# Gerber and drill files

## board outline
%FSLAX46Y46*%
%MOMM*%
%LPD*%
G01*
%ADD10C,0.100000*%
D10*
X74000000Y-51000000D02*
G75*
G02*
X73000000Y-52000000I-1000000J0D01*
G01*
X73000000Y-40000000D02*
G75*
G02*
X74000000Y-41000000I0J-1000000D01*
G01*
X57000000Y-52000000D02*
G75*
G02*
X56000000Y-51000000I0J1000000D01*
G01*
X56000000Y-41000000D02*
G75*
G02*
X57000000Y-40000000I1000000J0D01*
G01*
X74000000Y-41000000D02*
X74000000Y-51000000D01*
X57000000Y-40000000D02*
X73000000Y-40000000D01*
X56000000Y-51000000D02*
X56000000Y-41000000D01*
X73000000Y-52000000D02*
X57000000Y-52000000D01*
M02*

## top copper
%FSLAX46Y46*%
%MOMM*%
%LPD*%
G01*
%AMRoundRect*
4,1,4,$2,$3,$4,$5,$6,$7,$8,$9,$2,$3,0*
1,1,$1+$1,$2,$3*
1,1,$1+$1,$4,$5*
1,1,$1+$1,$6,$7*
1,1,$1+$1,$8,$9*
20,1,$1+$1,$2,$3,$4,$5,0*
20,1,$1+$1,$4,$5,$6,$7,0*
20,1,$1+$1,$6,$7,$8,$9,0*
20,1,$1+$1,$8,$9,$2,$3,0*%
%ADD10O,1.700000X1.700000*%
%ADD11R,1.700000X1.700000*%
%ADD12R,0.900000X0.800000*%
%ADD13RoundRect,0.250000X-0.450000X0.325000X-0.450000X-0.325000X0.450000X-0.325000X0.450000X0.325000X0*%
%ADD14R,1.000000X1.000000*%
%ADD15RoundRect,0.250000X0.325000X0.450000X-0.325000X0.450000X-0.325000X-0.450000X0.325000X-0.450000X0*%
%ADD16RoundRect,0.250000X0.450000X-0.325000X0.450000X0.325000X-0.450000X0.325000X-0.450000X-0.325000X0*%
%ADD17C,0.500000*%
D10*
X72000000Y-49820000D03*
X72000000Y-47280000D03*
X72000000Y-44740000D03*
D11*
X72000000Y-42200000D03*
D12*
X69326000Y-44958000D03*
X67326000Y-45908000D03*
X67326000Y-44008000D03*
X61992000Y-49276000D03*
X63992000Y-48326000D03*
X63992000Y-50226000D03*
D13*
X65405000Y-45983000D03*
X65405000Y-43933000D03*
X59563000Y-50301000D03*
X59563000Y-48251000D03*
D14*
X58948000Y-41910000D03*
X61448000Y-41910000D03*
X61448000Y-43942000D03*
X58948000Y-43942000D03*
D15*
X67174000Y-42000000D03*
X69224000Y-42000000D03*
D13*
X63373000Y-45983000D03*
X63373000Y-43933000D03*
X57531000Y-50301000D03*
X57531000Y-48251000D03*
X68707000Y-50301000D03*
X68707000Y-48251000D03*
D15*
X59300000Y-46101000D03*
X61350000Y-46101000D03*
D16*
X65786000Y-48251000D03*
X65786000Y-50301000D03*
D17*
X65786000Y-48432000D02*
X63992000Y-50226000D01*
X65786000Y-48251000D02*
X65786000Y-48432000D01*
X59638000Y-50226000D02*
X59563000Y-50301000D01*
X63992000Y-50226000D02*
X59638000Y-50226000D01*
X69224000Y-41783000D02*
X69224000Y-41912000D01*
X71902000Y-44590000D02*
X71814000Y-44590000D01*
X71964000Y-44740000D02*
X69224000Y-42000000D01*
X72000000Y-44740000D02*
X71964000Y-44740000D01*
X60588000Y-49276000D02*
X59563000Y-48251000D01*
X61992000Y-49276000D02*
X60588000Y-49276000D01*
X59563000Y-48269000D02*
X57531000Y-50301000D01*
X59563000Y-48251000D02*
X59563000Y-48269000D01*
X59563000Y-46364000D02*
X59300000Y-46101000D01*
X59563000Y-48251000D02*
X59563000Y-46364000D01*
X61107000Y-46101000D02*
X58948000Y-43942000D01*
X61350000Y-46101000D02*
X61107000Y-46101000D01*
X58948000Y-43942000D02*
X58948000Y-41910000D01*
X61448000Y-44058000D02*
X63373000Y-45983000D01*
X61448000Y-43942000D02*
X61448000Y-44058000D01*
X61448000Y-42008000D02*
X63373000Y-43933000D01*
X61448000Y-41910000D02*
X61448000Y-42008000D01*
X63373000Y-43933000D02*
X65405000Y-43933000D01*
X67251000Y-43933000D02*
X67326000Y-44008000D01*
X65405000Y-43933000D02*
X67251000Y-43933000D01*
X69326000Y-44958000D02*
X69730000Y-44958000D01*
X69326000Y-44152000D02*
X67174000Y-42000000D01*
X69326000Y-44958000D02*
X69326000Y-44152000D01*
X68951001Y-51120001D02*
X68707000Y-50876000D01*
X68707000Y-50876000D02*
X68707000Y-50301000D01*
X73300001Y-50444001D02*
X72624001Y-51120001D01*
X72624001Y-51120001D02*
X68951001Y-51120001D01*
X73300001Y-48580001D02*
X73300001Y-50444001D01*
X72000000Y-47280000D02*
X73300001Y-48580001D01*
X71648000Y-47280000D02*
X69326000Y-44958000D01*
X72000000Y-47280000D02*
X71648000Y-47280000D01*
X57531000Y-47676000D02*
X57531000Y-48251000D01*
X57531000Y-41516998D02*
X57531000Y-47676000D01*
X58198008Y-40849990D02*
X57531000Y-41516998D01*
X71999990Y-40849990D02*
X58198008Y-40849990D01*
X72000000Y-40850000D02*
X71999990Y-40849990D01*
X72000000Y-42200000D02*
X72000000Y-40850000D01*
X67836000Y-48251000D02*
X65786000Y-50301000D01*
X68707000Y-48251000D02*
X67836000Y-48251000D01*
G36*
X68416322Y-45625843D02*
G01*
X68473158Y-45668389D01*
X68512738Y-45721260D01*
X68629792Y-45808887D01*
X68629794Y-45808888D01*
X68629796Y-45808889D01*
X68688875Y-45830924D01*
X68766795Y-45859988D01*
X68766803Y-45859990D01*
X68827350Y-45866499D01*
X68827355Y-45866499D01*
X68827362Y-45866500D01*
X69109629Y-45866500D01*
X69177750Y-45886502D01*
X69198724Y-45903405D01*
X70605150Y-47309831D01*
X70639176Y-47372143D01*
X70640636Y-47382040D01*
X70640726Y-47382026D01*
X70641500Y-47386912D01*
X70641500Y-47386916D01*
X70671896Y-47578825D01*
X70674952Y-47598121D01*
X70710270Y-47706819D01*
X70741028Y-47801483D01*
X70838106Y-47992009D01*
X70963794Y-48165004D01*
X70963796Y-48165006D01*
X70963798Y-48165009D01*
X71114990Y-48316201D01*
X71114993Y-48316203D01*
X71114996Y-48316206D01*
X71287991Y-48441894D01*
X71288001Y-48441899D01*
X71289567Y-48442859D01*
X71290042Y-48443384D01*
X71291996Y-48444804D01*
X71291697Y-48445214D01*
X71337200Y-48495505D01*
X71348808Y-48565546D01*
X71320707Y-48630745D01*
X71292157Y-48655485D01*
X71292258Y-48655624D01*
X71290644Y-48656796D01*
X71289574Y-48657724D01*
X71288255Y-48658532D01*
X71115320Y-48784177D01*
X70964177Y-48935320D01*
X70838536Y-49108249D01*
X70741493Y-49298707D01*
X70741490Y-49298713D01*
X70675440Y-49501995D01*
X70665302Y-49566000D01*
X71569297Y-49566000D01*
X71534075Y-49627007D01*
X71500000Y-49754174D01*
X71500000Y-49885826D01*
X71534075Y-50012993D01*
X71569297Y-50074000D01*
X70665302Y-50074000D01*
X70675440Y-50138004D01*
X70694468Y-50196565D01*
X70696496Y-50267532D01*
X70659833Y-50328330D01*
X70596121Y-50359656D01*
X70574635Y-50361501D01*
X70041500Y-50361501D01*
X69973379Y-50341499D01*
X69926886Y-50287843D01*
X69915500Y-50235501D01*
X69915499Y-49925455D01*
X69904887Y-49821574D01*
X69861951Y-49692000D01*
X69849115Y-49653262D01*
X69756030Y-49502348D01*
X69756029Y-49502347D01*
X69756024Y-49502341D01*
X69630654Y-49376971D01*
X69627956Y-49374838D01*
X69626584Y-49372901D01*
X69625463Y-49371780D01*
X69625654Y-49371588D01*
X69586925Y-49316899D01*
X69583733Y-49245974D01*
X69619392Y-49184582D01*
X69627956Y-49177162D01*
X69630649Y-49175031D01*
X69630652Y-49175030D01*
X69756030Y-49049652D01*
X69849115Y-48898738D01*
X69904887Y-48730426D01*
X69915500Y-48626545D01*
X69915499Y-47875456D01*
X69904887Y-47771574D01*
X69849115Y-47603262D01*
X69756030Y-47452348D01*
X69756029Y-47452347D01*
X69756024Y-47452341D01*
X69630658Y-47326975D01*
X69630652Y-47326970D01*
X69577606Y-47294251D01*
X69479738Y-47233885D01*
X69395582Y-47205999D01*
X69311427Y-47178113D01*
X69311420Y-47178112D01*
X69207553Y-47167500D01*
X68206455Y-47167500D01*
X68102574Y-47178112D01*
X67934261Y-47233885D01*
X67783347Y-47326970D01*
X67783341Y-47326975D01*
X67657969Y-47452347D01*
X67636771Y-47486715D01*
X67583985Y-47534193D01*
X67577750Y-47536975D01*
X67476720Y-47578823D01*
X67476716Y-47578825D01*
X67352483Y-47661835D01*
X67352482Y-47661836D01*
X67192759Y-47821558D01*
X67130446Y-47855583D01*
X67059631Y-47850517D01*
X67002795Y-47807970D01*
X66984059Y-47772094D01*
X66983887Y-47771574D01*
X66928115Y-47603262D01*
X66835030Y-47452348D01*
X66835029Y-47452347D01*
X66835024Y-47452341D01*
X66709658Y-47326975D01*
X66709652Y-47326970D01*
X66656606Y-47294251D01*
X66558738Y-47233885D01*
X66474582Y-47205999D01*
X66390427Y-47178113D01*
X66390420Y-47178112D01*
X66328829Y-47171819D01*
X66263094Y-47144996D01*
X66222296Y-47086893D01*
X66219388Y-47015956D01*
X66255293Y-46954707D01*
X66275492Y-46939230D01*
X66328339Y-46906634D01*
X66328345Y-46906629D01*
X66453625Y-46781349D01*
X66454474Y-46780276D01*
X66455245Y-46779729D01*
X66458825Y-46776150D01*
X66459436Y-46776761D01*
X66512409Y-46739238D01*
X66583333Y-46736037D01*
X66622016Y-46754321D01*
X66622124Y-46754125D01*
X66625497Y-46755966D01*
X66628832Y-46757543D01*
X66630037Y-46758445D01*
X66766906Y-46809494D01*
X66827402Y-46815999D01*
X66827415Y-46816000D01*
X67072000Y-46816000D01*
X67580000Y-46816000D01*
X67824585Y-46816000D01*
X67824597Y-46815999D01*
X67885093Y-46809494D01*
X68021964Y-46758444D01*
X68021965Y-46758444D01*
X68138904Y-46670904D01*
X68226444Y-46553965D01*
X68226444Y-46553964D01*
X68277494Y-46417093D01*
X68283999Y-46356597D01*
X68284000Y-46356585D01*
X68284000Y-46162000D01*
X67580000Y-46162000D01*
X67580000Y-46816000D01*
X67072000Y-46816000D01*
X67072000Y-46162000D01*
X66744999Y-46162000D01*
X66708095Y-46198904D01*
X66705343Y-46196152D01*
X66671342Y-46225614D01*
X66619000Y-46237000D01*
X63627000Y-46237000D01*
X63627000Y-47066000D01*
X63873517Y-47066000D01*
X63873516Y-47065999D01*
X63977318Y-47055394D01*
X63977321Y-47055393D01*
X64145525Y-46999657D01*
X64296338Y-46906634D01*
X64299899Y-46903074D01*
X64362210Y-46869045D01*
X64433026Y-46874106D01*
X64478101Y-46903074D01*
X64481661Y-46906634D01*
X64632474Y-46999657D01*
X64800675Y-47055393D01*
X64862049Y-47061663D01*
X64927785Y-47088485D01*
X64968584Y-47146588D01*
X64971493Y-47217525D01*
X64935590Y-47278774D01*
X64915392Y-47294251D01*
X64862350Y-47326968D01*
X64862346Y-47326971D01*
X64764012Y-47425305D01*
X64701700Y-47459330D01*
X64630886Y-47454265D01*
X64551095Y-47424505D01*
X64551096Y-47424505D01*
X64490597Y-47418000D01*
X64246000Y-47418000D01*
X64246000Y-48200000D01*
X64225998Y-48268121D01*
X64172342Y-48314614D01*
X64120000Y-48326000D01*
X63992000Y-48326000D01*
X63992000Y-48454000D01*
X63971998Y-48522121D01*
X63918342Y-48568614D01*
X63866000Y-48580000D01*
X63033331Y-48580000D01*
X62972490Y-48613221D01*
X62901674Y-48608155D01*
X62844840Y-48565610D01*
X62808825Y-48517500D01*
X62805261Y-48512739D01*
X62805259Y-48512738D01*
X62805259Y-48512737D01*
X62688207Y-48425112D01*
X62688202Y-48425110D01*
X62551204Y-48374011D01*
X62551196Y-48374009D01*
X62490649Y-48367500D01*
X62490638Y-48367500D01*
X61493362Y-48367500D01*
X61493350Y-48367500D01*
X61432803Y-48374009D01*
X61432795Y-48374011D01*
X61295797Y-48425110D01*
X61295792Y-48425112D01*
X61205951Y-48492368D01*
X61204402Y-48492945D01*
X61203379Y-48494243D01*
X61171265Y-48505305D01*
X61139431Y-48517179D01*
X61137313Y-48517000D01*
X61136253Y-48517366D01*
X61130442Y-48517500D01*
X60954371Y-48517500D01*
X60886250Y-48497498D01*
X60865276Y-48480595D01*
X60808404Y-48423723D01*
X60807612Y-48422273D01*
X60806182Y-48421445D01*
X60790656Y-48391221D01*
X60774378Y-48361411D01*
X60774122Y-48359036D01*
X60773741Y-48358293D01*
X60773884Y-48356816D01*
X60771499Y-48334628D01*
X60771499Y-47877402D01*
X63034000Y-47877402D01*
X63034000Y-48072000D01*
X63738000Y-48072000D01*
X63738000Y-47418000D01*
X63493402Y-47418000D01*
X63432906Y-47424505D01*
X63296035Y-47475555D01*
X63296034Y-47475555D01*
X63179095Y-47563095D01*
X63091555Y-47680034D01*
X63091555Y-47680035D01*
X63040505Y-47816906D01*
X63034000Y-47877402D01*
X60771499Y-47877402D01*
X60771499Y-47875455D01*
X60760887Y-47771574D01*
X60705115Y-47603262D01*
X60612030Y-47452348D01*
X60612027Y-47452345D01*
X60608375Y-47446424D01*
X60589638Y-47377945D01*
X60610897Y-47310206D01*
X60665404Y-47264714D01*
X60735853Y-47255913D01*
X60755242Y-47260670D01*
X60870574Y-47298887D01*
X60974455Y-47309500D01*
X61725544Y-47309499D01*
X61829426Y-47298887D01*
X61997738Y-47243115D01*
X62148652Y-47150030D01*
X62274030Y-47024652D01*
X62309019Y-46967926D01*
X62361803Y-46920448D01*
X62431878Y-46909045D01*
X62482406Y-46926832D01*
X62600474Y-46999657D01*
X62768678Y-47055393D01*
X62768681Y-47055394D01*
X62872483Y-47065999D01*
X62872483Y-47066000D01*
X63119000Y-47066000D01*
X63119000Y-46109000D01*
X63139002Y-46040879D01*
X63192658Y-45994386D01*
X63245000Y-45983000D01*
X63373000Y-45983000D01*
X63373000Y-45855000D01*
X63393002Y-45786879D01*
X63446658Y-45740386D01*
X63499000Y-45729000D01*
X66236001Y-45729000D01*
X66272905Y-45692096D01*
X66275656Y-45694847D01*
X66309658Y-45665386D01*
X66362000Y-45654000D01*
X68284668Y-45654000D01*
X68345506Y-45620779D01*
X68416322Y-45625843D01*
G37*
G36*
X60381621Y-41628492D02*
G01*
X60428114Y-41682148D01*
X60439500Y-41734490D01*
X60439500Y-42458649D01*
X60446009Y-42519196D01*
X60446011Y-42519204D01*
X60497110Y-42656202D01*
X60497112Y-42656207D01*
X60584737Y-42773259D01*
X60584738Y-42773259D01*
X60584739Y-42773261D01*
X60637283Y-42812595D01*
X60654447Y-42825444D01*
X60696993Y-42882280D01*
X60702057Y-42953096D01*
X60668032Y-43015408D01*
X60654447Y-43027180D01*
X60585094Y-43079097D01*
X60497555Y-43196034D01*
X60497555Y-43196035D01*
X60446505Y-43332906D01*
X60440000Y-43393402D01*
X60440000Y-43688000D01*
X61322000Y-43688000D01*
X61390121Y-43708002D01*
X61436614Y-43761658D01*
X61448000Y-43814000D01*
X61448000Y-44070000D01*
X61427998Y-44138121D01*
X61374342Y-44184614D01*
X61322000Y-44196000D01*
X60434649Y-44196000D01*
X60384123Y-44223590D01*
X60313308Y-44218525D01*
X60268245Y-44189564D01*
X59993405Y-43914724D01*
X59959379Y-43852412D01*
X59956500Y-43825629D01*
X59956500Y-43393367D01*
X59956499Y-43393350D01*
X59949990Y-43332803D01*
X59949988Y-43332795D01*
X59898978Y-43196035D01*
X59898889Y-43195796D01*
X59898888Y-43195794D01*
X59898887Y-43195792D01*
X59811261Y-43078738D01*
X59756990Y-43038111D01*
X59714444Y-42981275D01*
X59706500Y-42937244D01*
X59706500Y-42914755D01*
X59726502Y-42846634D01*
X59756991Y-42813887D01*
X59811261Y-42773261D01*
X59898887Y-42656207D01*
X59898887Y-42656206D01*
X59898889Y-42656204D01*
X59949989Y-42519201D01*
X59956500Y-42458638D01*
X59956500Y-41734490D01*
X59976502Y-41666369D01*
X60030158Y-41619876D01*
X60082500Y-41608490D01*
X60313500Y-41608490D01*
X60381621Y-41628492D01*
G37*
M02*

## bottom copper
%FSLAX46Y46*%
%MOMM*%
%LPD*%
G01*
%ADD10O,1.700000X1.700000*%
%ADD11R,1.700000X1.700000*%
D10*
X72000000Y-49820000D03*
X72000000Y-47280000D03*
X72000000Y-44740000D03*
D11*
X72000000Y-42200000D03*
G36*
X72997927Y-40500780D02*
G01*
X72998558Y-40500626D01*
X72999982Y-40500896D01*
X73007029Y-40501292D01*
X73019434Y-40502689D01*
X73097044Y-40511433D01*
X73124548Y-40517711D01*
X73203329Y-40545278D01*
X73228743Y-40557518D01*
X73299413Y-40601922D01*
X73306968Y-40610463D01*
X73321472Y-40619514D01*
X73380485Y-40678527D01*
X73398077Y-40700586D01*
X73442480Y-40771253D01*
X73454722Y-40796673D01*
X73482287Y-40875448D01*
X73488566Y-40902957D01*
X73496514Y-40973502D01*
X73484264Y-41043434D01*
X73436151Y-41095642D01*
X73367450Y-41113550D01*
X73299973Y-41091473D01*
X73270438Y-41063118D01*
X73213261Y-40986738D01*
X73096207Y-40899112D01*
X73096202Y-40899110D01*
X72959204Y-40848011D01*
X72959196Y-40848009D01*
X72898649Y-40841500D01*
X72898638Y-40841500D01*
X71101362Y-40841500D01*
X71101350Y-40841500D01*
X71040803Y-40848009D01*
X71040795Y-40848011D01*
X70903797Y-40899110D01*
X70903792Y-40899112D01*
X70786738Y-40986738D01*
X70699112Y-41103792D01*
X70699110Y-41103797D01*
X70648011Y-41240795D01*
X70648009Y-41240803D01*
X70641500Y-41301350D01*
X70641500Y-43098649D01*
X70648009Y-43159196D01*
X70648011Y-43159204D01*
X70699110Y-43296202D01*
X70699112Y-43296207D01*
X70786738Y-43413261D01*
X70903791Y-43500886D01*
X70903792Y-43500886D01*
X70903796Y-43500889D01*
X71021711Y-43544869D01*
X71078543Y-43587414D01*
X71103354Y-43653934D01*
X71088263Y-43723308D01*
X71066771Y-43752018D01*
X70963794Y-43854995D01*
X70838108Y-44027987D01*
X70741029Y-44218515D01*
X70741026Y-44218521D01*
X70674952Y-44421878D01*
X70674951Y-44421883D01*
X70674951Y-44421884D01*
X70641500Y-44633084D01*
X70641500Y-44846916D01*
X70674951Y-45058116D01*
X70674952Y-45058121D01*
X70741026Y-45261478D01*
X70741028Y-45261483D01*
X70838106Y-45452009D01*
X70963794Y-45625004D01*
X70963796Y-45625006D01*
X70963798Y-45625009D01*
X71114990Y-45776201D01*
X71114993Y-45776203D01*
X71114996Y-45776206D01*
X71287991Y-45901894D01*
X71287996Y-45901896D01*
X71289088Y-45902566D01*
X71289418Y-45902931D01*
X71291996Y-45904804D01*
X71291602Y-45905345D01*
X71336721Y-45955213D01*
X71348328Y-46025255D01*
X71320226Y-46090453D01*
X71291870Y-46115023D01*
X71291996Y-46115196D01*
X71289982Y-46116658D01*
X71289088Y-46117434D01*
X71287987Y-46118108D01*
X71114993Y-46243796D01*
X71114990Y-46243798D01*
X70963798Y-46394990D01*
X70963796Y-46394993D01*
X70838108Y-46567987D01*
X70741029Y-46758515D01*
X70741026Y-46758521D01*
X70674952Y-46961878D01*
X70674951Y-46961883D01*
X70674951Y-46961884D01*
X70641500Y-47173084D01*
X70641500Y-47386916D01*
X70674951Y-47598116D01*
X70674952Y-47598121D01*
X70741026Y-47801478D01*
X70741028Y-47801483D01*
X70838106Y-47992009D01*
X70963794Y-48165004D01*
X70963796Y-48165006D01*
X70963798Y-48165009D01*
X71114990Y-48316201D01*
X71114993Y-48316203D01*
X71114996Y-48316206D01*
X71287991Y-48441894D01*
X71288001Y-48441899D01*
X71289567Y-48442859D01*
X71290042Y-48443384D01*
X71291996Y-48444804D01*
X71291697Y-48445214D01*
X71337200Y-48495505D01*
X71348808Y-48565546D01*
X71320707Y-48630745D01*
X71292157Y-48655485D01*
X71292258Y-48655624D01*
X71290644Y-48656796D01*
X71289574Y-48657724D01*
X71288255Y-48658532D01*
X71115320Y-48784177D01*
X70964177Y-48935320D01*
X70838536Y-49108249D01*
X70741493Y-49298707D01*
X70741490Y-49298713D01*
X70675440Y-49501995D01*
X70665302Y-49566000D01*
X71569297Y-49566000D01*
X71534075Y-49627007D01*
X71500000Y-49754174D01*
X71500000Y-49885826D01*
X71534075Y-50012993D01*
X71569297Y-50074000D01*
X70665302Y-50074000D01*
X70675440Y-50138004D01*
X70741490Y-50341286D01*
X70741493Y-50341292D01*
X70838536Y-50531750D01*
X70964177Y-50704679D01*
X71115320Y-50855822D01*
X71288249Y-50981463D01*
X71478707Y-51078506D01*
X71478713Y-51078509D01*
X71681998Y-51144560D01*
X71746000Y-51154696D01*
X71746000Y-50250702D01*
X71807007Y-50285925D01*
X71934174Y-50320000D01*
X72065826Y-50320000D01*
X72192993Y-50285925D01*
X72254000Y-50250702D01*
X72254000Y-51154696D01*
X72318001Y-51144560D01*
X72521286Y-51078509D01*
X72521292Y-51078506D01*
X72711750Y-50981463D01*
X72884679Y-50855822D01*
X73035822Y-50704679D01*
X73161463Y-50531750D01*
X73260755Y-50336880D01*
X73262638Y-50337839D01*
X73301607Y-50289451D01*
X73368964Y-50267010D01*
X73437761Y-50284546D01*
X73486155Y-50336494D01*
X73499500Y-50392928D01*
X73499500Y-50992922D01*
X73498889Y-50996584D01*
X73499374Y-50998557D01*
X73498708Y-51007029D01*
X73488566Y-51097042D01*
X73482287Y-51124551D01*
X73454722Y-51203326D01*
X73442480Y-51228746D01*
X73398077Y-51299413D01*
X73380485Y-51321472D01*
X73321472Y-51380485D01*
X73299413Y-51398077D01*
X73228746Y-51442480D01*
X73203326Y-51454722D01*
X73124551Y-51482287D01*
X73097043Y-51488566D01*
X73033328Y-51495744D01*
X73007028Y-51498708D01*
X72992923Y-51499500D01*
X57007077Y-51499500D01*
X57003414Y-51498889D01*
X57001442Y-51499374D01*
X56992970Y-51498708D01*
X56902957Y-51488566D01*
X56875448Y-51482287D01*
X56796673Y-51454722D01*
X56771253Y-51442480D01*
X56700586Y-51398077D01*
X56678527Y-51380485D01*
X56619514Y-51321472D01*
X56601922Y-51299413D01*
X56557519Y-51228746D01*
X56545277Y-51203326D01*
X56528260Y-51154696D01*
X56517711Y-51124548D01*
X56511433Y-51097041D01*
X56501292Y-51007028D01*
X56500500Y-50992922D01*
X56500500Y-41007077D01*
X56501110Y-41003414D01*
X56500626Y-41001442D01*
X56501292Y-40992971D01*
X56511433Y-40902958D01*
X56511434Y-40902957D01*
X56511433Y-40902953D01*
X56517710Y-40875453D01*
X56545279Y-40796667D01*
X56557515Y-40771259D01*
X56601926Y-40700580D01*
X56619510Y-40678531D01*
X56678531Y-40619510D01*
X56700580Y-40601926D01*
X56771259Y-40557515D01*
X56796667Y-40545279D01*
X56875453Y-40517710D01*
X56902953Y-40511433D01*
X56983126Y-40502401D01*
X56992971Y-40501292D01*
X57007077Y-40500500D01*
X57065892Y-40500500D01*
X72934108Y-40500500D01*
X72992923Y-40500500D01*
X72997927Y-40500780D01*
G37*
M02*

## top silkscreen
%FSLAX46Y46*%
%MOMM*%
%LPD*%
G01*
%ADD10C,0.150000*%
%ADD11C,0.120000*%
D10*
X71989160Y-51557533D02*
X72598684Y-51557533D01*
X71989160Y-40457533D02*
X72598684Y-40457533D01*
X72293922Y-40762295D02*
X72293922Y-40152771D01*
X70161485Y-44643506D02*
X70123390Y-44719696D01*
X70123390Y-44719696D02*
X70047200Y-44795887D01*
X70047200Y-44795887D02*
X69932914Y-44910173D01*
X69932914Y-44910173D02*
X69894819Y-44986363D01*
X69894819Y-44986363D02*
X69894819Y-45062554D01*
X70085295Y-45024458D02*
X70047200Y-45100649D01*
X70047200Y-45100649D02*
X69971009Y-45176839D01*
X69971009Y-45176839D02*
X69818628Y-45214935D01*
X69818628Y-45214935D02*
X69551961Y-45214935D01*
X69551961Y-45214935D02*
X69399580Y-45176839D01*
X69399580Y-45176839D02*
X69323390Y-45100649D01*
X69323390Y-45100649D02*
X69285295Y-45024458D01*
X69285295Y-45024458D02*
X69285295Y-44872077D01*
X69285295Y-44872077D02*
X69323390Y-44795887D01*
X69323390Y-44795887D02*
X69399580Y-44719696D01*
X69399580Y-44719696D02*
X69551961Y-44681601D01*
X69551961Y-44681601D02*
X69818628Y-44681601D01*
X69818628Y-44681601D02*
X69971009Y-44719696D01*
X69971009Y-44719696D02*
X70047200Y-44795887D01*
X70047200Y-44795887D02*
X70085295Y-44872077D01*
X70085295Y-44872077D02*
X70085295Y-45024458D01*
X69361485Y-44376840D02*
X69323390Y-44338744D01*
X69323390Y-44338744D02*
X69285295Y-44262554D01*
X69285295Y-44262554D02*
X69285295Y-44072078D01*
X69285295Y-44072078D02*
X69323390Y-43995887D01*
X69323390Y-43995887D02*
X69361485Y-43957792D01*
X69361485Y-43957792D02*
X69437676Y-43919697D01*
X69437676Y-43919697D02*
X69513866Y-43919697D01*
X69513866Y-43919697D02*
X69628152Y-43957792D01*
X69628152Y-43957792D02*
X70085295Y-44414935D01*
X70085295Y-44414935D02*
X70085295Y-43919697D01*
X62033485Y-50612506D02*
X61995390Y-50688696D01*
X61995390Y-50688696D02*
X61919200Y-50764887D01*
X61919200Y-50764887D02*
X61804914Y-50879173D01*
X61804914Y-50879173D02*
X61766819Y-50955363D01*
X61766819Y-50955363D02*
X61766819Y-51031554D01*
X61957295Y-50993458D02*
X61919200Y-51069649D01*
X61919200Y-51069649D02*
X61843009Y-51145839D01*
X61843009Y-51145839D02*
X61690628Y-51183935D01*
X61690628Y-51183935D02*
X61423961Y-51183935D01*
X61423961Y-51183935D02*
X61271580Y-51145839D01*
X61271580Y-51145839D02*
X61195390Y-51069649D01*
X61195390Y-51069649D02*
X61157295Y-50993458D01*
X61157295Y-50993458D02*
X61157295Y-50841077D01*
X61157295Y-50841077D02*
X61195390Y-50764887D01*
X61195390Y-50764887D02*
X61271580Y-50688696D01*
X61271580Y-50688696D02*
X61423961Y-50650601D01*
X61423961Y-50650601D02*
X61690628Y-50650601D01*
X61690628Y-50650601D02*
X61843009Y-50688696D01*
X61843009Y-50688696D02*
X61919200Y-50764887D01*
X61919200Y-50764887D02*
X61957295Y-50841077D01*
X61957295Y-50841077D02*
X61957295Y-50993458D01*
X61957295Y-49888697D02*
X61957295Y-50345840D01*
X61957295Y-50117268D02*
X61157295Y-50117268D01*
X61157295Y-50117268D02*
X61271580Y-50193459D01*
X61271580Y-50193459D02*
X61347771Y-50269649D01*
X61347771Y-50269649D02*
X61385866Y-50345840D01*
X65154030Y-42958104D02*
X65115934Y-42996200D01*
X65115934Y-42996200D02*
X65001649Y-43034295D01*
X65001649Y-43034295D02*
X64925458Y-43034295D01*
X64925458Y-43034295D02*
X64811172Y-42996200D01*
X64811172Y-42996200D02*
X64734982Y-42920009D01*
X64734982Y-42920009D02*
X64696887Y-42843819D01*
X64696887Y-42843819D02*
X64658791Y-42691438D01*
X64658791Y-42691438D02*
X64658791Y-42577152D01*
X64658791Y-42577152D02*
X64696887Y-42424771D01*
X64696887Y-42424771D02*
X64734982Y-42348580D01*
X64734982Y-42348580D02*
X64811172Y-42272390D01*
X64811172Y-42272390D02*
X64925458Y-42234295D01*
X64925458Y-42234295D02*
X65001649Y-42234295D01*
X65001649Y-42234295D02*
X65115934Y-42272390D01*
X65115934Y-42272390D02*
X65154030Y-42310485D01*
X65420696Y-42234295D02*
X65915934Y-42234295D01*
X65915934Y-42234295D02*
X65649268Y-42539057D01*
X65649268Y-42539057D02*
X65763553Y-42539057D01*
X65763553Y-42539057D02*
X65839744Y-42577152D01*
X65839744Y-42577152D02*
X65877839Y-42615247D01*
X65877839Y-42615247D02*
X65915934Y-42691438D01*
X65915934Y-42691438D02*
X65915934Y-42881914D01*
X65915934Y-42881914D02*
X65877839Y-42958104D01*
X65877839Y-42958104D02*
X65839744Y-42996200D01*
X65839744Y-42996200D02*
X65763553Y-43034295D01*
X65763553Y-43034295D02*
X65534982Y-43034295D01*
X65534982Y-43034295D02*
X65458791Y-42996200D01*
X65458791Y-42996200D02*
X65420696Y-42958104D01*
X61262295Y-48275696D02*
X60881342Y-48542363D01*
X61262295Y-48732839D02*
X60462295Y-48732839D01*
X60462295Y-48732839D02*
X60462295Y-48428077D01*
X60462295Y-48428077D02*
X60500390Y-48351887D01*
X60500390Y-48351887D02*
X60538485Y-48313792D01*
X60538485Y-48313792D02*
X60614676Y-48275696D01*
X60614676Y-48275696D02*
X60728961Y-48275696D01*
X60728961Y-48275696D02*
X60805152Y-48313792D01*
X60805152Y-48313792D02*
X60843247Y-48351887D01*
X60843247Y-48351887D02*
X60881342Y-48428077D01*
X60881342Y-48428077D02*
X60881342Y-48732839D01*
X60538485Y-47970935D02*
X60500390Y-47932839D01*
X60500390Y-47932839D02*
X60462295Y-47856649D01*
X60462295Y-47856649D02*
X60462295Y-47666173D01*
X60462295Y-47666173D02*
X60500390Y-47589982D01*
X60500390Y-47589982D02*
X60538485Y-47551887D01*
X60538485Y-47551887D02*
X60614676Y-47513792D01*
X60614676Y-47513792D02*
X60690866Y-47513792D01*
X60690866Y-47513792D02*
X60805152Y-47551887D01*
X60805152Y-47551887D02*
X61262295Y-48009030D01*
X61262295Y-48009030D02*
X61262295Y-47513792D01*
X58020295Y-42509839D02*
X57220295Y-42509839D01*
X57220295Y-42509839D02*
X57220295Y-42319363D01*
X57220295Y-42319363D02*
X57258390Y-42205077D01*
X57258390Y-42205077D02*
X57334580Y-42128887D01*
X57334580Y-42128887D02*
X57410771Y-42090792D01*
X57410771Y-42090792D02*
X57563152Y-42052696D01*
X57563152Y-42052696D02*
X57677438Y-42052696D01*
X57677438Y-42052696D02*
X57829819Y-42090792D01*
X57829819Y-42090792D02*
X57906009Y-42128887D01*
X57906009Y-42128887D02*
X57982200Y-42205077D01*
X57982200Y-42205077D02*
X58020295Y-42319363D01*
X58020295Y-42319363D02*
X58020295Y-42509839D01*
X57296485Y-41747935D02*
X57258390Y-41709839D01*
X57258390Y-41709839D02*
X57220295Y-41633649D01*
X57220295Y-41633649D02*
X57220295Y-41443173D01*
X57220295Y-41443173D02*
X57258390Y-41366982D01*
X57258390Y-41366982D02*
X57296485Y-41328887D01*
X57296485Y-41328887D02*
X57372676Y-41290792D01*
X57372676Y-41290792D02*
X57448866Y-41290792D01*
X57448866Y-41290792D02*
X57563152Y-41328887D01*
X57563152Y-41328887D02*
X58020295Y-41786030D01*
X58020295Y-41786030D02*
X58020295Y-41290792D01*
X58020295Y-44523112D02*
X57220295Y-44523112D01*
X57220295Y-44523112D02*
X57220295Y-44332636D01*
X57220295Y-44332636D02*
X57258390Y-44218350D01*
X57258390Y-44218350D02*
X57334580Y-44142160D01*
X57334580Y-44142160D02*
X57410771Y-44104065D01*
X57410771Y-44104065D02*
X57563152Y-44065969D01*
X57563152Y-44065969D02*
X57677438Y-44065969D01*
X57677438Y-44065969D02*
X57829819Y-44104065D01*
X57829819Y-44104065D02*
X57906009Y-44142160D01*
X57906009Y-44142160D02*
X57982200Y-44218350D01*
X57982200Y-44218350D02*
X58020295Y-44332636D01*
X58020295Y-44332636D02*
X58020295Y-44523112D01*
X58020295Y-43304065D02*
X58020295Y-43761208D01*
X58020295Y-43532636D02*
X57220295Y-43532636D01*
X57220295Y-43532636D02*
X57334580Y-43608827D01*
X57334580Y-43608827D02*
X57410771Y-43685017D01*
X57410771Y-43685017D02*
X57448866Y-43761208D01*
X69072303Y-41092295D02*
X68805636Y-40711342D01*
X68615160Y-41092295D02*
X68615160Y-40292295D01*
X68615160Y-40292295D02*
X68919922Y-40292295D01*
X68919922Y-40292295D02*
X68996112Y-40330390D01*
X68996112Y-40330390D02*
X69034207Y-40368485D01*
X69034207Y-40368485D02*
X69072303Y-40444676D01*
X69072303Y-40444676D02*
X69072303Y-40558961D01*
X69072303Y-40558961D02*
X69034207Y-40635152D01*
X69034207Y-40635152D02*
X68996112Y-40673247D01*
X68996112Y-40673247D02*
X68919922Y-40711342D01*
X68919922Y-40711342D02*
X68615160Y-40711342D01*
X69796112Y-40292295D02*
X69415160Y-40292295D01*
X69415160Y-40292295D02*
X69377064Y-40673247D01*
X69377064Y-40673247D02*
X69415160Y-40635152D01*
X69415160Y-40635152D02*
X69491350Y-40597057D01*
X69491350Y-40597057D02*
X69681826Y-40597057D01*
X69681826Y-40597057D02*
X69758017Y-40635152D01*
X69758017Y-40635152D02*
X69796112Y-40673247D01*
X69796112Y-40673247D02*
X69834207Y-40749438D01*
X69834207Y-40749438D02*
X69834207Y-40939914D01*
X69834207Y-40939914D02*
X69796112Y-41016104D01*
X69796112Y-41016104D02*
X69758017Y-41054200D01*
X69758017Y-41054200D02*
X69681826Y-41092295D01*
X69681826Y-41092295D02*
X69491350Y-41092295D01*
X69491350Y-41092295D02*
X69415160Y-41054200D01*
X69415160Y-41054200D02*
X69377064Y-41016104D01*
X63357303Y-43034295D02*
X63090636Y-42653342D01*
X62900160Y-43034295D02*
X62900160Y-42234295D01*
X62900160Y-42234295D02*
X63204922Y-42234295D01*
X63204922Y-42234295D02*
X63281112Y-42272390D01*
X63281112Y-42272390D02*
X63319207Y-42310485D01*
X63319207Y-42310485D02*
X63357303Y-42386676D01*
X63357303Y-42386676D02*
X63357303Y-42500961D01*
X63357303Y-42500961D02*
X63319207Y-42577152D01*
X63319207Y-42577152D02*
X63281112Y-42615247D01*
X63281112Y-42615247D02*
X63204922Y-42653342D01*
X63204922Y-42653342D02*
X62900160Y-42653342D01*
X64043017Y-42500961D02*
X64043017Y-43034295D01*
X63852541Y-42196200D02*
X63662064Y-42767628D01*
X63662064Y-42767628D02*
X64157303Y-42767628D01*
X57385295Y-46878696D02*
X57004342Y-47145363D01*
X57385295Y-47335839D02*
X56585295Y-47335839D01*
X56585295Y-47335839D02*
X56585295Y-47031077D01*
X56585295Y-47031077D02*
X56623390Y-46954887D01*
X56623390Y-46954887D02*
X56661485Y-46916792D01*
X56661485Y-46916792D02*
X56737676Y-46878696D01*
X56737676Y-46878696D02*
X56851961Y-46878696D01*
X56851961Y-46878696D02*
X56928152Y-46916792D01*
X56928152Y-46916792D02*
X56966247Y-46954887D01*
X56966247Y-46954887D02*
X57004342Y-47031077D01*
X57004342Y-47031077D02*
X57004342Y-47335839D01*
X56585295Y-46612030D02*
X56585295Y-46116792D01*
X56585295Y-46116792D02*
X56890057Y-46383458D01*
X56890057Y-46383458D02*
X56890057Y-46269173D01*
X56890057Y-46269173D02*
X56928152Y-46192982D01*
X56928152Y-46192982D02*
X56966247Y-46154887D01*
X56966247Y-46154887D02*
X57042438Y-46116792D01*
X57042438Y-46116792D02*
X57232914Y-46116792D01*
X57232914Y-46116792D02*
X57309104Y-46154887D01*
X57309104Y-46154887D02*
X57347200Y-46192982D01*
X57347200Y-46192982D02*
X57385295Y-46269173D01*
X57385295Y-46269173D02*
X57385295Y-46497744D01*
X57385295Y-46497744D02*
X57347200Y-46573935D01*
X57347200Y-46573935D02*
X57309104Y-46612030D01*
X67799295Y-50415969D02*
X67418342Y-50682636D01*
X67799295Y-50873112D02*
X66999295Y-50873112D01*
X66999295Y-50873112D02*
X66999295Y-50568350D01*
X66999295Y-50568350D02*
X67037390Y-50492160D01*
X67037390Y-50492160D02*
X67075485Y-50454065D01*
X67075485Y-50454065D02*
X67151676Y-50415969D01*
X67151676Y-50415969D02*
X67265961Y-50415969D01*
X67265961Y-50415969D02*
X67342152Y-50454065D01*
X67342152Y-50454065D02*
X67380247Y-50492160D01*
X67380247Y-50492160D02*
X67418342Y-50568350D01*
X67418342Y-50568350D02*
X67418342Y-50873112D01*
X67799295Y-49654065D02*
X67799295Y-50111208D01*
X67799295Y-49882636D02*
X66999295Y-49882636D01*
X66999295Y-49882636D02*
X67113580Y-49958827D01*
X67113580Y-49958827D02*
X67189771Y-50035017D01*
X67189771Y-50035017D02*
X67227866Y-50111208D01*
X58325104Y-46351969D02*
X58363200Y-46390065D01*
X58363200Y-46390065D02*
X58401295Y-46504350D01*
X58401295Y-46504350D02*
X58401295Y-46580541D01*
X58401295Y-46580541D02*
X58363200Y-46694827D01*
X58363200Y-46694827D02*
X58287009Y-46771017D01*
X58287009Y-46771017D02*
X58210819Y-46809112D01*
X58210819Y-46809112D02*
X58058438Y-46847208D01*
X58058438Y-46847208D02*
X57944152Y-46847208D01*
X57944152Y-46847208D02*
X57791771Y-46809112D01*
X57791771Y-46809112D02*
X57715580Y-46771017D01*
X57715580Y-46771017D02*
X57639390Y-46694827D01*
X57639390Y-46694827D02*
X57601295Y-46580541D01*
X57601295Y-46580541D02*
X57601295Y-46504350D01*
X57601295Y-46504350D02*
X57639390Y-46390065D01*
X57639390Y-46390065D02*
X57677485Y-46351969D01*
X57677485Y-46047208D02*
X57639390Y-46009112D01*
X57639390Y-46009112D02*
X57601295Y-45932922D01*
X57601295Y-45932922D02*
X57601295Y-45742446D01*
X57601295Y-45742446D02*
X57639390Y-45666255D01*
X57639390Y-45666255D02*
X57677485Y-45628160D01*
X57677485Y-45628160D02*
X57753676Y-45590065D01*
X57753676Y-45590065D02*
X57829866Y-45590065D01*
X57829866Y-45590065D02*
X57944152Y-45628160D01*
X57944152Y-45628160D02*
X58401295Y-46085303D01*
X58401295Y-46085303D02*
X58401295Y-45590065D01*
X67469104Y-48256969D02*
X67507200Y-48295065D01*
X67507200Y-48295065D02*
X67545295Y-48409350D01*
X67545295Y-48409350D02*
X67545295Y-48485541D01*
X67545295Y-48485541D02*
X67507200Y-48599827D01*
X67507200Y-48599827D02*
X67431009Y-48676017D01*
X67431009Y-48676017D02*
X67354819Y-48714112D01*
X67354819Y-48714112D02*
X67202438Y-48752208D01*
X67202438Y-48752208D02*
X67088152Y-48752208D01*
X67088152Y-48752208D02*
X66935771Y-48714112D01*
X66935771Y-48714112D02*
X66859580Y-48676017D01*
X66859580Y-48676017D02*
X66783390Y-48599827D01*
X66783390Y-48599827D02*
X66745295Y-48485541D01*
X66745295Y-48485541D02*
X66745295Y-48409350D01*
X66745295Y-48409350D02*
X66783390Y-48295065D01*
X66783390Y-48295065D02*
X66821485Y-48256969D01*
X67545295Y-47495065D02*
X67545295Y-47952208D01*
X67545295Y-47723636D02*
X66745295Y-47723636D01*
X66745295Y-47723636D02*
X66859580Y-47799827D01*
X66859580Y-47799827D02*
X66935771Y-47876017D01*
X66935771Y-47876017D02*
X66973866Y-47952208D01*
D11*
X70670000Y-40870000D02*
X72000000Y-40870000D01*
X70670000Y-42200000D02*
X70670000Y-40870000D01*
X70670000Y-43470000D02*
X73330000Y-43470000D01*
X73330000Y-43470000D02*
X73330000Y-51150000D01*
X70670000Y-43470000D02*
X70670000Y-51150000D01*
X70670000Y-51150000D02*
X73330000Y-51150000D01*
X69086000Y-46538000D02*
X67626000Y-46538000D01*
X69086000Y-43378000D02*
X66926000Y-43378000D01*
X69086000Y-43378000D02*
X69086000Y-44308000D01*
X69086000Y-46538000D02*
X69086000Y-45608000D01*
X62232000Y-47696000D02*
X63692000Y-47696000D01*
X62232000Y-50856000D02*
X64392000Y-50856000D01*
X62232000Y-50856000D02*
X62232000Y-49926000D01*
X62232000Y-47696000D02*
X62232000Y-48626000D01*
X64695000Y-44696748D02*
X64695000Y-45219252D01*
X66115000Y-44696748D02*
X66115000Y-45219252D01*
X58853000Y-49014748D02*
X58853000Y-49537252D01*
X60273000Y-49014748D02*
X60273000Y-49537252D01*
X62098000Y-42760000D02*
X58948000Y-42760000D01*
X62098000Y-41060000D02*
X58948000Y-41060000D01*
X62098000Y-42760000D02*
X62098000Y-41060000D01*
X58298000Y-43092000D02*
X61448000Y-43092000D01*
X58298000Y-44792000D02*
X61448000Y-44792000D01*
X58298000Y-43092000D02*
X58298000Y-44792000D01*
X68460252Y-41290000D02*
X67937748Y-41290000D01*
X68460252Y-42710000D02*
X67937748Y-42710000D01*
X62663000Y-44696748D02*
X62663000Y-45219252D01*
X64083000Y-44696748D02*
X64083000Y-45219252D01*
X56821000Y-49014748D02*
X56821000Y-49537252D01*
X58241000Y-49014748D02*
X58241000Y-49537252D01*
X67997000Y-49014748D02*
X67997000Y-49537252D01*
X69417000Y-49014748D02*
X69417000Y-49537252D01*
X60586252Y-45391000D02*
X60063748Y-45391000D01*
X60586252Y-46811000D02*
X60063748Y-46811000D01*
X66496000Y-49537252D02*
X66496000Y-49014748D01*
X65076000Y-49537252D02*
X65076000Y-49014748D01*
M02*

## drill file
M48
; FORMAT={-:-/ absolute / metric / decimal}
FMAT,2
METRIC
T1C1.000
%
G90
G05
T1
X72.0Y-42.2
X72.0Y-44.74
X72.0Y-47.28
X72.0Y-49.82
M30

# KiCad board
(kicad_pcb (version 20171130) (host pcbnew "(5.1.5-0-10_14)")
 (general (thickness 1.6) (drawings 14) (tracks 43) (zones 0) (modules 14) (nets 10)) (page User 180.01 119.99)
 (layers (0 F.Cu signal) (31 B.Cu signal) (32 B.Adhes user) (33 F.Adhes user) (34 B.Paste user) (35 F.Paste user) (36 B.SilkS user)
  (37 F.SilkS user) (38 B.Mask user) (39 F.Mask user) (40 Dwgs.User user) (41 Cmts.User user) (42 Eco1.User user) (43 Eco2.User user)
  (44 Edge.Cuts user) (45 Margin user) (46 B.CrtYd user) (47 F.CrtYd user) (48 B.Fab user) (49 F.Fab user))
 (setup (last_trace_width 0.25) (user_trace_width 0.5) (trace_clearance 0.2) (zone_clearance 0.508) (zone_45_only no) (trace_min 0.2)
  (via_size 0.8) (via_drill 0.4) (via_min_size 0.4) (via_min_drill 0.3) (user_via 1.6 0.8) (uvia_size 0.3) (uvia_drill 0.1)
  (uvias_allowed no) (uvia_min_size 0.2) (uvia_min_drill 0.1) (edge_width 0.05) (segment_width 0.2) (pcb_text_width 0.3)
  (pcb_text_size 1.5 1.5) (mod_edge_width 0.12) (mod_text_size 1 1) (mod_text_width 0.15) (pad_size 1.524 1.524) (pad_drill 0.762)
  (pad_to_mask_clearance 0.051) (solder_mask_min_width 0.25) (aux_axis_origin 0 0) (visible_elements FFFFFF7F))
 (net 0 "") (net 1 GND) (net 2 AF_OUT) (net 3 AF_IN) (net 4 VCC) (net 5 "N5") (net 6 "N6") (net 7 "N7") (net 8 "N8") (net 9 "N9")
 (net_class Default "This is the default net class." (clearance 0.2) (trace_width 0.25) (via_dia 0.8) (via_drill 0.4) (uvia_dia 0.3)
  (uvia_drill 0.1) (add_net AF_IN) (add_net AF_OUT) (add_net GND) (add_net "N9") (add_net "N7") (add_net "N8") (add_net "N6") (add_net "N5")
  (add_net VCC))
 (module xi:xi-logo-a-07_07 (layer B.Cu) (at 61.5 46 270)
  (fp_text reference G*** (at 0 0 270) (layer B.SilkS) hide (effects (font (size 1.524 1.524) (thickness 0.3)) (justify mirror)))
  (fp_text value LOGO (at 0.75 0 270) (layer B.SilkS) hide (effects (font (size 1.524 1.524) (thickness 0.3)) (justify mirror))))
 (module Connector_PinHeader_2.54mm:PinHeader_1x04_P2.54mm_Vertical (layer F.Cu) (at 72 42.2)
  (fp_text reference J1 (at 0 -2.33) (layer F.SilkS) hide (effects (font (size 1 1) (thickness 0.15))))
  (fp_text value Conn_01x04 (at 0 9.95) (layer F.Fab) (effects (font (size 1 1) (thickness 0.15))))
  (fp_line (start -1.33 -1.33) (end 0 -1.33) (layer F.SilkS) (width 0.12))
  (fp_line (start -1.33 0) (end -1.33 -1.33) (layer F.SilkS) (width 0.12))
  (fp_line (start -1.33 1.27) (end 1.33 1.27) (layer F.SilkS) (width 0.12))
  (fp_line (start 1.33 1.27) (end 1.33 8.95) (layer F.SilkS) (width 0.12))
  (fp_line (start -1.33 1.27) (end -1.33 8.95) (layer F.SilkS) (width 0.12))
  (fp_line (start -1.33 8.95) (end 1.33 8.95) (layer F.SilkS) (width 0.12))
  (pad 4 thru_hole oval (at 0 7.62) (size 1.7 1.7) (drill 1) (layers *.Cu *.Mask) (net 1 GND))
  (pad 3 thru_hole oval (at 0 5.08) (size 1.7 1.7) (drill 1) (layers *.Cu *.Mask) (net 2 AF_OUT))
  (pad 2 thru_hole oval (at 0 2.54) (size 1.7 1.7) (drill 1) (layers *.Cu *.Mask) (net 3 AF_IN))
  (pad 1 thru_hole rect (at 0 0) (size 1.7 1.7) (drill 1) (layers *.Cu *.Mask) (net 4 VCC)))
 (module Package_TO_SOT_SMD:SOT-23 (layer F.Cu) (at 68.326 44.958)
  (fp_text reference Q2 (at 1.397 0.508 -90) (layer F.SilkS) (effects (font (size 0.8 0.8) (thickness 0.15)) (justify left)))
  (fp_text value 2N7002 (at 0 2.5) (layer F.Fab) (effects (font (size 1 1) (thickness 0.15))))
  (fp_line (start 0.76 1.58) (end -0.7 1.58) (layer F.SilkS) (width 0.12))
  (fp_line (start 0.76 -1.58) (end -1.4 -1.58) (layer F.SilkS) (width 0.12))
  (fp_line (start 0.76 -1.58) (end 0.76 -0.65) (layer F.SilkS) (width 0.12))
  (fp_line (start 0.76 1.58) (end 0.76 0.65) (layer F.SilkS) (width 0.12))
  (pad 3 smd rect (at 1 0) (size 0.9 0.8) (layers F.Cu F.Paste F.Mask) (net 2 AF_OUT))
  (pad 2 smd rect (at -1 0.95) (size 0.9 0.8) (layers F.Cu F.Paste F.Mask) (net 1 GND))
  (pad 1 smd rect (at -1 -0.95) (size 0.9 0.8) (layers F.Cu F.Paste F.Mask) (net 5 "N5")))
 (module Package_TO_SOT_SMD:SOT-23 (layer F.Cu) (at 62.992 49.276 180)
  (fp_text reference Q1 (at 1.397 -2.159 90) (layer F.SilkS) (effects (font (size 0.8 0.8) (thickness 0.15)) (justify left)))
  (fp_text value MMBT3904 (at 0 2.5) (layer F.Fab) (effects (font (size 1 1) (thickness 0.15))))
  (fp_line (start 0.76 1.58) (end -0.7 1.58) (layer F.SilkS) (width 0.12))
  (fp_line (start 0.76 -1.58) (end -1.4 -1.58) (layer F.SilkS) (width 0.12))
  (fp_line (start 0.76 -1.58) (end 0.76 -0.65) (layer F.SilkS) (width 0.12))
  (fp_line (start 0.76 1.58) (end 0.76 0.65) (layer F.SilkS) (width 0.12))
  (pad 3 smd rect (at 1 0 180) (size 0.9 0.8) (layers F.Cu F.Paste F.Mask) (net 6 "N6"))
  (pad 2 smd rect (at -1 0.95 180) (size 0.9 0.8) (layers F.Cu F.Paste F.Mask) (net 1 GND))
  (pad 1 smd rect (at -1 -0.95 180) (size 0.9 0.8) (layers F.Cu F.Paste F.Mask) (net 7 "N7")))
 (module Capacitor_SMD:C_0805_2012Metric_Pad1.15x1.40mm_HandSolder (layer F.Cu) (at 65.405 44.958 270)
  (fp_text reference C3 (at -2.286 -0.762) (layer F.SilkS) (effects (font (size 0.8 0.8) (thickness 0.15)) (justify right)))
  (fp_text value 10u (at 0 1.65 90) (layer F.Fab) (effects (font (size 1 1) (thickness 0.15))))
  (fp_line (start -0.261252 0.71) (end 0.261252 0.71) (layer F.SilkS) (width 0.12))
  (fp_line (start -0.261252 -0.71) (end 0.261252 -0.71) (layer F.SilkS) (width 0.12))
  (pad 2 smd roundrect (at 1.025 0 270) (size 1.15 1.4) (layers F.Cu F.Paste F.Mask) (roundrect_rratio 0.217391) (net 1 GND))
  (pad 1 smd roundrect (at -1.025 0 270) (size 1.15 1.4) (layers F.Cu F.Paste F.Mask) (roundrect_rratio 0.217391) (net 5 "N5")))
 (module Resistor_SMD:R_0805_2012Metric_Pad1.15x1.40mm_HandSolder (layer F.Cu) (at 59.563 49.276 270)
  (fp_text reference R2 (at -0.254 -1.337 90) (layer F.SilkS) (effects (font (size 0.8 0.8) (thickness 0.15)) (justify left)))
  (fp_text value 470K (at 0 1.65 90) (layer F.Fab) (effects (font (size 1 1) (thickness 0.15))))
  (fp_line (start -0.261252 0.71) (end 0.261252 0.71) (layer F.SilkS) (width 0.12))
  (fp_line (start -0.261252 -0.71) (end 0.261252 -0.71) (layer F.SilkS) (width 0.12))
  (pad 2 smd roundrect (at 1.025 0 270) (size 1.15 1.4) (layers F.Cu F.Paste F.Mask) (roundrect_rratio 0.217391) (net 7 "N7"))
  (pad 1 smd roundrect (at -1.025 0 270) (size 1.15 1.4) (layers F.Cu F.Paste F.Mask) (roundrect_rratio 0.217391) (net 6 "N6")))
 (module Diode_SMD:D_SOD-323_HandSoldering (layer F.Cu) (at 60.198 41.91 180)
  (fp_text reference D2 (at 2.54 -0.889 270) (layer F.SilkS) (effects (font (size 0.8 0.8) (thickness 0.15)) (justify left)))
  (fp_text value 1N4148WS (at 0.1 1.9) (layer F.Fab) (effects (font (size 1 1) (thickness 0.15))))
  (fp_line (start -1.9 -0.85) (end 1.25 -0.85) (layer F.SilkS) (width 0.12))
  (fp_line (start -1.9 0.85) (end 1.25 0.85) (layer F.SilkS) (width 0.12))
  (fp_line (start -1.9 -0.85) (end -1.9 0.85) (layer F.SilkS) (width 0.12))
  (pad 2 smd rect (at 1.25 0 180) (size 1 1) (layers F.Cu F.Paste F.Mask) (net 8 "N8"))
  (pad 1 smd rect (at -1.25 0 180) (size 1 1) (layers F.Cu F.Paste F.Mask) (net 5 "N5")))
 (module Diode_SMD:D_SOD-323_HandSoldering (layer F.Cu) (at 60.198 43.942)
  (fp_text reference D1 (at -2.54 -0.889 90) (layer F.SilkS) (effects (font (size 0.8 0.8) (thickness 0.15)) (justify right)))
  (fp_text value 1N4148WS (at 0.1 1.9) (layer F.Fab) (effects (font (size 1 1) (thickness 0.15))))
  (fp_line (start -1.9 -0.85) (end 1.25 -0.85) (layer F.SilkS) (width 0.12))
  (fp_line (start -1.9 0.85) (end 1.25 0.85) (layer F.SilkS) (width 0.12))
  (fp_line (start -1.9 -0.85) (end -1.9 0.85) (layer F.SilkS) (width 0.12))
  (pad 2 smd rect (at 1.25 0) (size 1 1) (layers F.Cu F.Paste F.Mask) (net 1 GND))
  (pad 1 smd rect (at -1.25 0) (size 1 1) (layers F.Cu F.Paste F.Mask) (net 8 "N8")))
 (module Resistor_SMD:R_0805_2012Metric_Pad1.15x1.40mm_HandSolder (layer F.Cu) (at 68.199 42 180)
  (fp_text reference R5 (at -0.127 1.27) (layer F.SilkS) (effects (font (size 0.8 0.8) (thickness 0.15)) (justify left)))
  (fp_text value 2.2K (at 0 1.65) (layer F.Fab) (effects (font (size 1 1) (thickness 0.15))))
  (fp_line (start -0.261252 0.71) (end 0.261252 0.71) (layer F.SilkS) (width 0.12))
  (fp_line (start -0.261252 -0.71) (end 0.261252 -0.71) (layer F.SilkS) (width 0.12))
  (pad 2 smd roundrect (at 1.025 0 180) (size 1.15 1.4) (layers F.Cu F.Paste F.Mask) (roundrect_rratio 0.217391) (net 2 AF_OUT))
  (pad 1 smd roundrect (at -1.025 0 180) (size 1.15 1.4) (layers F.Cu F.Paste F.Mask) (roundrect_rratio 0.217391) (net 3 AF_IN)))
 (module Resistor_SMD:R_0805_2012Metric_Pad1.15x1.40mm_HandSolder (layer F.Cu) (at 63.373 44.958 270)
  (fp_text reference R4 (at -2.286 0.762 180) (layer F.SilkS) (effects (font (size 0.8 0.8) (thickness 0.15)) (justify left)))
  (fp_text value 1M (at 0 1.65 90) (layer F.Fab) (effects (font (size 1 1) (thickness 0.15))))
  (fp_line (start -0.261252 0.71) (end 0.261252 0.71) (layer F.SilkS) (width 0.12))
  (fp_line (start -0.261252 -0.71) (end 0.261252 -0.71) (layer F.SilkS) (width 0.12))
  (pad 2 smd roundrect (at 1.025 0 270) (size 1.15 1.4) (layers F.Cu F.Paste F.Mask) (roundrect_rratio 0.217391) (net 1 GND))
  (pad 1 smd roundrect (at -1.025 0 270) (size 1.15 1.4) (layers F.Cu F.Paste F.Mask) (roundrect_rratio 0.217391) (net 5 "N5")))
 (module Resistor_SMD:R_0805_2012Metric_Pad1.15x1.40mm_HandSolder (layer F.Cu) (at 57.531 49.276 270)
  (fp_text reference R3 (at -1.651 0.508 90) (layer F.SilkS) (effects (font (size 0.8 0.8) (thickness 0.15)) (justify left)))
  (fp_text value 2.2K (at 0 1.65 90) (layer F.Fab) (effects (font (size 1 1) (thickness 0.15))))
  (fp_line (start -0.261252 0.71) (end 0.261252 0.71) (layer F.SilkS) (width 0.12))
  (fp_line (start -0.261252 -0.71) (end 0.261252 -0.71) (layer F.SilkS) (width 0.12))
  (pad 2 smd roundrect (at 1.025 0 270) (size 1.15 1.4) (layers F.Cu F.Paste F.Mask) (roundrect_rratio 0.217391) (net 6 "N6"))
  (pad 1 smd roundrect (at -1.025 0 270) (size 1.15 1.4) (layers F.Cu F.Paste F.Mask) (roundrect_rratio 0.217391) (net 4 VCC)))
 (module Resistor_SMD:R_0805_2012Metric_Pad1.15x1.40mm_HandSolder (layer F.Cu) (at 68.707 49.276 270)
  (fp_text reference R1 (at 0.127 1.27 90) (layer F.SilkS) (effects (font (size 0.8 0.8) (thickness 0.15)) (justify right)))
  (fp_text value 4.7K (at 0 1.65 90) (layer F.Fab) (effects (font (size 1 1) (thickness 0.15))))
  (fp_line (start -0.261252 0.71) (end 0.261252 0.71) (layer F.SilkS) (width 0.12))
  (fp_line (start -0.261252 -0.71) (end 0.261252 -0.71) (layer F.SilkS) (width 0.12))
  (pad 2 smd roundrect (at 1.025 0 270) (size 1.15 1.4) (layers F.Cu F.Paste F.Mask) (roundrect_rratio 0.217391) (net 2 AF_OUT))
  (pad 1 smd roundrect (at -1.025 0 270) (size 1.15 1.4) (layers F.Cu F.Paste F.Mask) (roundrect_rratio 0.217391) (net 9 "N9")))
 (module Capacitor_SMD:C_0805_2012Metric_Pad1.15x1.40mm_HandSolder (layer F.Cu) (at 60.325 46.101 180)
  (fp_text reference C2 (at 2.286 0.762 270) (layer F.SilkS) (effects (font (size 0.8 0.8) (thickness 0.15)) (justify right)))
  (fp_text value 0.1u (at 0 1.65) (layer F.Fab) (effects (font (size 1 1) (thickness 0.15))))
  (fp_line (start -0.261252 0.71) (end 0.261252 0.71) (layer F.SilkS) (width 0.12))
  (fp_line (start -0.261252 -0.71) (end 0.261252 -0.71) (layer F.SilkS) (width 0.12))
  (pad 2 smd roundrect (at 1.025 0 180) (size 1.15 1.4) (layers F.Cu F.Paste F.Mask) (roundrect_rratio 0.217391) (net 6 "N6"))
  (pad 1 smd roundrect (at -1.025 0 180) (size 1.15 1.4) (layers F.Cu F.Paste F.Mask) (roundrect_rratio 0.217391) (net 8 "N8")))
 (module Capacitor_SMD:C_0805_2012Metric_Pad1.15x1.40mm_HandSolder (layer F.Cu) (at 65.786 49.276 90)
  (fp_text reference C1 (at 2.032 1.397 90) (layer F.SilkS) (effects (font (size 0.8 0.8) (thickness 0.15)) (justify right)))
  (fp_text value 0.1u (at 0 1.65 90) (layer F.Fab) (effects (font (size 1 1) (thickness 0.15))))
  (fp_line (start -0.261252 0.71) (end 0.261252 0.71) (layer F.SilkS) (width 0.12))
  (fp_line (start -0.261252 -0.71) (end 0.261252 -0.71) (layer F.SilkS) (width 0.12))
  (pad 2 smd roundrect (at 1.025 0 90) (size 1.15 1.4) (layers F.Cu F.Paste F.Mask) (roundrect_rratio 0.217391) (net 7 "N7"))
  (pad 1 smd roundrect (at -1.025 0 90) (size 1.15 1.4) (layers F.Cu F.Paste F.Mask) (roundrect_rratio 0.217391) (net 9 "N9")))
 (gr_arc (start 73 51) (end 73 52) (angle -90) (layer Edge.Cuts) (width 0.1))
 (gr_arc (start 73 41) (end 74 41) (angle -90) (layer Edge.Cuts) (width 0.1))
 (gr_arc (start 57 51) (end 56 51) (angle -90) (layer Edge.Cuts) (width 0.1))
 (gr_arc (start 57 41) (end 57 40) (angle -90) (layer Edge.Cuts) (width 0.1))
 (gr_line (start 74 41) (end 74 51) (layer Edge.Cuts) (width 0.1))
 (gr_line (start 57 40) (end 73 40) (layer Edge.Cuts) (width 0.1))
 (gr_line (start 56 51) (end 56 41) (layer Edge.Cuts) (width 0.1))
 (gr_line (start 73 52) (end 57 52) (layer Edge.Cuts) (width 0.1))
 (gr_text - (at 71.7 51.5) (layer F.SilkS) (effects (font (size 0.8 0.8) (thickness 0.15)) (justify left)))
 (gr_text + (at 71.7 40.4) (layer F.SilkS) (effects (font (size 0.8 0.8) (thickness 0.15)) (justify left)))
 (segment (start 65.786 48.432) (end 63.992 50.226) (width 0.5) (layer F.Cu) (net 7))
 (segment (start 65.786 48.251) (end 65.786 48.432) (width 0.5) (layer F.Cu) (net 7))
 (segment (start 59.638 50.226) (end 59.563 50.301) (width 0.5) (layer F.Cu) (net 7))
 (segment (start 63.992 50.226) (end 59.638 50.226) (width 0.5) (layer F.Cu) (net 7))
 (segment (start 69.224 41.783) (end 69.224 41.912) (width 0.5) (layer F.Cu) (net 3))
 (segment (start 71.902 44.59) (end 71.814 44.59) (width 0.5) (layer F.Cu) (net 3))
 (segment (start 71.964 44.74) (end 69.224 42) (width 0.5) (layer F.Cu) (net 3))
 (segment (start 72 44.74) (end 71.964 44.74) (width 0.5) (layer F.Cu) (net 3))
 (segment (start 60.588 49.276) (end 59.563 48.251) (width 0.5) (layer F.Cu) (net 6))
 (segment (start 61.992 49.276) (end 60.588 49.276) (width 0.5) (layer F.Cu) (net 6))
 (segment (start 59.563 48.269) (end 57.531 50.301) (width 0.5) (layer F.Cu) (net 6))
 (segment (start 59.563 48.251) (end 59.563 48.269) (width 0.5) (layer F.Cu) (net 6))
 (segment (start 59.563 46.364) (end 59.3 46.101) (width 0.5) (layer F.Cu) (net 6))
 (segment (start 59.563 48.251) (end 59.563 46.364) (width 0.5) (layer F.Cu) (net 6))
 (segment (start 61.107 46.101) (end 58.948 43.942) (width 0.5) (layer F.Cu) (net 8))
 (segment (start 61.35 46.101) (end 61.107 46.101) (width 0.5) (layer F.Cu) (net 8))
 (segment (start 58.948 43.942) (end 58.948 41.91) (width 0.5) (layer F.Cu) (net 8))
 (segment (start 61.448 44.058) (end 63.373 45.983) (width 0.5) (layer F.Cu) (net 1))
 (segment (start 61.448 43.942) (end 61.448 44.058) (width 0.5) (layer F.Cu) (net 1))
 (segment (start 61.448 42.008) (end 63.373 43.933) (width 0.5) (layer F.Cu) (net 5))
 (segment (start 61.448 41.91) (end 61.448 42.008) (width 0.5) (layer F.Cu) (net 5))
 (segment (start 63.373 43.933) (end 65.405 43.933) (width 0.5) (layer F.Cu) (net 5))
 (segment (start 67.251 43.933) (end 67.326 44.008) (width 0.5) (layer F.Cu) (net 5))
 (segment (start 65.405 43.933) (end 67.251 43.933) (width 0.5) (layer F.Cu) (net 5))
 (segment (start 69.326 44.958) (end 69.73 44.958) (width 0.5) (layer F.Cu) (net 2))
 (segment (start 69.326 44.152) (end 67.174 42) (width 0.5) (layer F.Cu) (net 2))
 (segment (start 69.326 44.958) (end 69.326 44.152) (width 0.5) (layer F.Cu) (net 2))
 (segment (start 68.951001 51.120001) (end 68.707 50.876) (width 0.5) (layer F.Cu) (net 2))
 (segment (start 68.707 50.876) (end 68.707 50.301) (width 0.5) (layer F.Cu) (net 2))
 (segment (start 73.300001 50.444001) (end 72.624001 51.120001) (width 0.5) (layer F.Cu) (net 2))
 (segment (start 72.624001 51.120001) (end 68.951001 51.120001) (width 0.5) (layer F.Cu) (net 2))
 (segment (start 73.300001 48.580001) (end 73.300001 50.444001) (width 0.5) (layer F.Cu) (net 2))
 (segment (start 72 47.28) (end 73.300001 48.580001) (width 0.5) (layer F.Cu) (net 2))
 (segment (start 71.648 47.28) (end 69.326 44.958) (width 0.5) (layer F.Cu) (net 2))
 (segment (start 72 47.28) (end 71.648 47.28) (width 0.5) (layer F.Cu) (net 2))
 (segment (start 57.531 47.676) (end 57.531 48.251) (width 0.5) (layer F.Cu) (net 4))
 (segment (start 57.531 41.516998) (end 57.531 47.676) (width 0.5) (layer F.Cu) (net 4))
 (segment (start 58.198008 40.84999) (end 57.531 41.516998) (width 0.5) (layer F.Cu) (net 4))
 (segment (start 71.99999 40.84999) (end 58.198008 40.84999) (width 0.5) (layer F.Cu) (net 4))
 (segment (start 72 40.85) (end 71.99999 40.84999) (width 0.5) (layer F.Cu) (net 4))
 (segment (start 72 42.2) (end 72 40.85) (width 0.5) (layer F.Cu) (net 4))
 (segment (start 67.836 48.251) (end 65.786 50.301) (width 0.5) (layer F.Cu) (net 9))
 (segment (start 68.707 48.251) (end 67.836 48.251) (width 0.5) (layer F.Cu) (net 9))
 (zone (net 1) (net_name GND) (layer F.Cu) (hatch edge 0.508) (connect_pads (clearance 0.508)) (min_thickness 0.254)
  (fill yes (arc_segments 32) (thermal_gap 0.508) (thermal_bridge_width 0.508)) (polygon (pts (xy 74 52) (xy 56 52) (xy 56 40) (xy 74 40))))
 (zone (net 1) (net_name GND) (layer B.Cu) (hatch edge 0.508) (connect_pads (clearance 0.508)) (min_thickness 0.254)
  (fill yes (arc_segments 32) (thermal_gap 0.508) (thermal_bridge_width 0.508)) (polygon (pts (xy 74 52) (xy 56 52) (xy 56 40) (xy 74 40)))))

